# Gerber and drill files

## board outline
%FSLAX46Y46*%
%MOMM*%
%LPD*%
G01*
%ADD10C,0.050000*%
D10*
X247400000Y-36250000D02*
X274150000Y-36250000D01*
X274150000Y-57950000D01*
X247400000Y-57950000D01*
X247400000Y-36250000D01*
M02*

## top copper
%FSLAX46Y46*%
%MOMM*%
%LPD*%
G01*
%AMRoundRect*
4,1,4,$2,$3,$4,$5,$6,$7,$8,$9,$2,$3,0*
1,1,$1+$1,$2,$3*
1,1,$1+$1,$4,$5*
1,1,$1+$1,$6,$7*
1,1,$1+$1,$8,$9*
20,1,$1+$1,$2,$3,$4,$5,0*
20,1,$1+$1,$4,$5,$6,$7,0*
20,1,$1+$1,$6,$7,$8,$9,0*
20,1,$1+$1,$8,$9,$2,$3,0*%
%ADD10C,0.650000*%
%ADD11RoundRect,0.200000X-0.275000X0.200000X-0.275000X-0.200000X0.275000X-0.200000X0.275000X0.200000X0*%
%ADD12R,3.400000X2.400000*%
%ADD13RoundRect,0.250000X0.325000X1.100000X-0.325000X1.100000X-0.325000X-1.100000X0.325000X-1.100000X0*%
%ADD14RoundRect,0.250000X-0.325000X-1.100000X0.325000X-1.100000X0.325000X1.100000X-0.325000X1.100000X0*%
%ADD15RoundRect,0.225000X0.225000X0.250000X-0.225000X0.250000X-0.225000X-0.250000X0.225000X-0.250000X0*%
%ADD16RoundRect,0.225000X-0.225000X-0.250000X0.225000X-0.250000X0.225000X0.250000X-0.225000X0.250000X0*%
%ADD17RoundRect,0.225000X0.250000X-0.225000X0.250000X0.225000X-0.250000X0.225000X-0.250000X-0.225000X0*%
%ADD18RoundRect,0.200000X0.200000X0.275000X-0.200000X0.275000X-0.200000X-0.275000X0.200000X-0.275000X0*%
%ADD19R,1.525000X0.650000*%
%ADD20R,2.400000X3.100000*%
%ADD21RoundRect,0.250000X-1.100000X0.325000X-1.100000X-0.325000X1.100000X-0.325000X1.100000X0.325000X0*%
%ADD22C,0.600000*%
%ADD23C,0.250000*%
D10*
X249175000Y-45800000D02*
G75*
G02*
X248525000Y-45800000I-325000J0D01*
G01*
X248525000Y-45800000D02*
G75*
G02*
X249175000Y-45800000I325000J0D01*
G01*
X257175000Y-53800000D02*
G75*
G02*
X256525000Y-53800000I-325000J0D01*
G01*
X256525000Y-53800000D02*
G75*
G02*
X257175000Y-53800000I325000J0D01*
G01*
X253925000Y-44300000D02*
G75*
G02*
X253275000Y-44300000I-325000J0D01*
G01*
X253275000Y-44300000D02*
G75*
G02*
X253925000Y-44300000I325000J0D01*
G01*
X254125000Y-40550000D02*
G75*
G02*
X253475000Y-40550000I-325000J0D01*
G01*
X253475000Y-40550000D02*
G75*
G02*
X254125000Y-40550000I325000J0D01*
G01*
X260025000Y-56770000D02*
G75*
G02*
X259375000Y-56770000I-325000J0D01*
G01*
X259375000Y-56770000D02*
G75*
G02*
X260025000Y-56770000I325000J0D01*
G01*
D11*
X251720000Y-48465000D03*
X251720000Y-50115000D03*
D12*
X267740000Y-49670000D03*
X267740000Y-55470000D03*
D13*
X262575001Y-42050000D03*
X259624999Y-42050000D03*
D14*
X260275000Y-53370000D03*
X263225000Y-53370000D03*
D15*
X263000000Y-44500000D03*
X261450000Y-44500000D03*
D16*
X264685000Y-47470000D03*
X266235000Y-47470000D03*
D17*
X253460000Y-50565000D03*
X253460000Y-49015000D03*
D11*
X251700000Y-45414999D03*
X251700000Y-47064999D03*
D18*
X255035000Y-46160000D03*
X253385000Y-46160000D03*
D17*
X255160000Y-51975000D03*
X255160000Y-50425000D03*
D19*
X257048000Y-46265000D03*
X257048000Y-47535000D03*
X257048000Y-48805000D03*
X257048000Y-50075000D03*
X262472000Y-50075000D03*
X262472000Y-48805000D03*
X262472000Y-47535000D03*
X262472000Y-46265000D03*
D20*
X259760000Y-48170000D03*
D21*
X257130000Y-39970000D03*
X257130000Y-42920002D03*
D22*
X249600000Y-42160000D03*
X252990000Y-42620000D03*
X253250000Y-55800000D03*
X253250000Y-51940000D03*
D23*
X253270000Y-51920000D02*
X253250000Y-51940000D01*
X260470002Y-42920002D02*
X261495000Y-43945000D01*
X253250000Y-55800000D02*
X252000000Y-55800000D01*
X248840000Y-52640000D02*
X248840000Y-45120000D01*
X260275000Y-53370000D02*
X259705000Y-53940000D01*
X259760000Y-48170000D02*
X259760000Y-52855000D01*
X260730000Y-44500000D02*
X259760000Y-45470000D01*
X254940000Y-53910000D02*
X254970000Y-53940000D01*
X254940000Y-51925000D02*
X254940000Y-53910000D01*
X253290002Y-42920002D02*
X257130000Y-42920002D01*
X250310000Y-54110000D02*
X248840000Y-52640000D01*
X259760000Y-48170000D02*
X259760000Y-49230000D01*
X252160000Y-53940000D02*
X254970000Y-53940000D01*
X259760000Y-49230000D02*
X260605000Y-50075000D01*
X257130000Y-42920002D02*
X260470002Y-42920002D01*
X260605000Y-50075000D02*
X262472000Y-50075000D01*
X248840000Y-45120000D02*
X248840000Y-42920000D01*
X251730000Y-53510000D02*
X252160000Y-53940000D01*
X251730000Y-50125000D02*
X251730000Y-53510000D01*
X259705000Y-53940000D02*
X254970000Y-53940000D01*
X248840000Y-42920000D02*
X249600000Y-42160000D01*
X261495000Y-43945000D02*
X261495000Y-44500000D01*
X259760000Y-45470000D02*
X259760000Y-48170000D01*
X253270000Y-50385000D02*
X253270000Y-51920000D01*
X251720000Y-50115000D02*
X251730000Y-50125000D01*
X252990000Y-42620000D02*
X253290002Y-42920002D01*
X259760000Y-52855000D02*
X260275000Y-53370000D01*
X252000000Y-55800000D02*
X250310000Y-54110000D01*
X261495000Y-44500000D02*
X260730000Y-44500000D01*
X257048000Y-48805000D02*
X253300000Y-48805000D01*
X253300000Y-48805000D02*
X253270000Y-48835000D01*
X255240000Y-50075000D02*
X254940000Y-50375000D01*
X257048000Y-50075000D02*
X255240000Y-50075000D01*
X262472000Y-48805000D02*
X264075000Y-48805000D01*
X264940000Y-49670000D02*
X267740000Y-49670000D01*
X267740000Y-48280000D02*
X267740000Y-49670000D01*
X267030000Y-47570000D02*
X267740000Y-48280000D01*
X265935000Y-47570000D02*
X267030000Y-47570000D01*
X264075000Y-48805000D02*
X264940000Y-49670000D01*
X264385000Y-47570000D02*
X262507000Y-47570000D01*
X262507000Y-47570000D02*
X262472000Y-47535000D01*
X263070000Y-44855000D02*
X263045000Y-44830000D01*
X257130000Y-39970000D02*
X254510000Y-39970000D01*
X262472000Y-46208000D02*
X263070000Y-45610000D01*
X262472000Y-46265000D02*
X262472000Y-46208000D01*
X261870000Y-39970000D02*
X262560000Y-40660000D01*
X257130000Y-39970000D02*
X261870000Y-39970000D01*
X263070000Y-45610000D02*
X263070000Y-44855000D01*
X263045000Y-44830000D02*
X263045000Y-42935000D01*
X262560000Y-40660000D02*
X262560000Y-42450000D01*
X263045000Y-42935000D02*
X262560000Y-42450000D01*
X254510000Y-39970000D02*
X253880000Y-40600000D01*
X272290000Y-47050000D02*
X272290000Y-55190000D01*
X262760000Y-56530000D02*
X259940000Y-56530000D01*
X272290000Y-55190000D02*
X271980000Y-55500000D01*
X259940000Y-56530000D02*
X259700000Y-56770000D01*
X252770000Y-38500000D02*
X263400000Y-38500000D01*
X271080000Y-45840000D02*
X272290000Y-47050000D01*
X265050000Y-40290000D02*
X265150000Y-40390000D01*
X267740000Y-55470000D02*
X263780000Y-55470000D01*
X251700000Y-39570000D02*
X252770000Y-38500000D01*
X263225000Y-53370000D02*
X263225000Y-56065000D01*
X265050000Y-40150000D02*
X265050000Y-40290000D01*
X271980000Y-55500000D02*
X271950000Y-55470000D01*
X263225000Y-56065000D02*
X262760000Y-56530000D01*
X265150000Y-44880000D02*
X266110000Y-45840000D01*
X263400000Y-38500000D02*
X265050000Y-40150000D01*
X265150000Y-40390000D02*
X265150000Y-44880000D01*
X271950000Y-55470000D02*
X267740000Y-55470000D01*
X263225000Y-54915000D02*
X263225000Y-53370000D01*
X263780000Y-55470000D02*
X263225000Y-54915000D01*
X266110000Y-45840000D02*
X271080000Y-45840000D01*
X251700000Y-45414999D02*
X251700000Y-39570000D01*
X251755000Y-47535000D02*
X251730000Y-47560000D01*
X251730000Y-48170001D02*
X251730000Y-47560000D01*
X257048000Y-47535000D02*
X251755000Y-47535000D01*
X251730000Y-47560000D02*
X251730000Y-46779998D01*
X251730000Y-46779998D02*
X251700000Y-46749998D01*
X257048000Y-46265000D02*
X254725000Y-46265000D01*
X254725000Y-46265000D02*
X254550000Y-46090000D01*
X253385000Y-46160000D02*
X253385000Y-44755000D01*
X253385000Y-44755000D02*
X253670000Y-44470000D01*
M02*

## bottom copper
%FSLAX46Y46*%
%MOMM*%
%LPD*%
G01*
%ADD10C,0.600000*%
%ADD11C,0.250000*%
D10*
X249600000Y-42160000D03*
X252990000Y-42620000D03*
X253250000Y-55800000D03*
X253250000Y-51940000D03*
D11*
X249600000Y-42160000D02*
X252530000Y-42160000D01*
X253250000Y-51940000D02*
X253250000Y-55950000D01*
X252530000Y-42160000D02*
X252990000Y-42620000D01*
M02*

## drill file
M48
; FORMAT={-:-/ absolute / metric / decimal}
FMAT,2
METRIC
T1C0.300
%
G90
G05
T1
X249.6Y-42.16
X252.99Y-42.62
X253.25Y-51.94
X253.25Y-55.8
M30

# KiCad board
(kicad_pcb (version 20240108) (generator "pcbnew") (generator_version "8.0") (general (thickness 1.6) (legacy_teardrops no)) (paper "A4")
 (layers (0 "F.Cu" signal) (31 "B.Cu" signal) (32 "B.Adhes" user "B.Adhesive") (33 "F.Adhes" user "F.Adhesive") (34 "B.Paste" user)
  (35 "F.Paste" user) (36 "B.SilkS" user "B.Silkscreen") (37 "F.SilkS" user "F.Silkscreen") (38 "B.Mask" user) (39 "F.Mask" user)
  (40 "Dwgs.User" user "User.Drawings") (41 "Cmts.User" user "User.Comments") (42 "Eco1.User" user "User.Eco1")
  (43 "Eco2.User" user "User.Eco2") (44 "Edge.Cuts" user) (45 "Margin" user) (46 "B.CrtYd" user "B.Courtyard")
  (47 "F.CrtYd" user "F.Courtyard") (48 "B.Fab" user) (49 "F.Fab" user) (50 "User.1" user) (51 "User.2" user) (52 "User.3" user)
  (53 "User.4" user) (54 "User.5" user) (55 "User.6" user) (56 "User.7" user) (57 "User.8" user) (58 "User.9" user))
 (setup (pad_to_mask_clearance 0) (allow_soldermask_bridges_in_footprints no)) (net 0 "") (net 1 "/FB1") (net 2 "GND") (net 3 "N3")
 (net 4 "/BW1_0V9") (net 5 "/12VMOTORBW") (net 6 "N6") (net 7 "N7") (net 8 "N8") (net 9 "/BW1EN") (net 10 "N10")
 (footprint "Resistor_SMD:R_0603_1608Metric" (layer "F.Cu") (at 251.72 49.29 -90)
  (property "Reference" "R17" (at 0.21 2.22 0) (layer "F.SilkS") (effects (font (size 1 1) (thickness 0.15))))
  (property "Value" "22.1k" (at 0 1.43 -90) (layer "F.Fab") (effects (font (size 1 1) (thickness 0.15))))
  (pad "1" smd roundrect (at -0.825 0 270) (size 0.8 0.95) (layers "F.Cu" "F.Paste" "F.Mask") (roundrect_rratio 0.25) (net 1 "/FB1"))
  (pad "2" smd roundrect (at 0.825 0 270) (size 0.8 0.95) (layers "F.Cu" "F.Paste" "F.Mask") (roundrect_rratio 0.25) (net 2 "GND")))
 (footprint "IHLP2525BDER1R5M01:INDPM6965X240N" (layer "F.Cu") (at 267.74 52.57 -90)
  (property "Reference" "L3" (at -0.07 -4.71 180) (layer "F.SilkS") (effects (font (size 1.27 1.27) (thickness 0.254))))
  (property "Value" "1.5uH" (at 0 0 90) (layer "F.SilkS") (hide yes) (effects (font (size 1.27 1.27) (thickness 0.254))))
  (pad "1" smd rect (at -2.9 0 270) (size 2.4 3.4) (layers "F.Cu" "F.Paste" "F.Mask") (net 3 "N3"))
  (pad "2" smd rect (at 2.9 0 270) (size 2.4 3.4) (layers "F.Cu" "F.Paste" "F.Mask") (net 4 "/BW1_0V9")))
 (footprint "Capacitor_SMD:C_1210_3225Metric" (layer "F.Cu") (at 261.1 42.05 180)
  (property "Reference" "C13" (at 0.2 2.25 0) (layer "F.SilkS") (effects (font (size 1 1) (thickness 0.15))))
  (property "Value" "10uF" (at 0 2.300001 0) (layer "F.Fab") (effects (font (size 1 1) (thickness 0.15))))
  (pad "1" smd roundrect (at -1.475001 0 180) (size 1.15 2.7) (layers "F.Cu" "F.Paste" "F.Mask") (roundrect_rratio 0.217391)
   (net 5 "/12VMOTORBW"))
  (pad "2" smd roundrect (at 1.475001 0 180) (size 1.15 2.7) (layers "F.Cu" "F.Paste" "F.Mask") (roundrect_rratio 0.217391) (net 2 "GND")))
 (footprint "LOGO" (layer "F.Cu") (at 268.9 41.65)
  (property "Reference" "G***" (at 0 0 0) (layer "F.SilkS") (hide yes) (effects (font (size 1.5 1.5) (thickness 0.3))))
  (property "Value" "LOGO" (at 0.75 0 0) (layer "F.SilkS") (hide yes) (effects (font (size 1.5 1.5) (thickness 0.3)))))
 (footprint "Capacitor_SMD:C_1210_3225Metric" (layer "F.Cu") (at 261.75 53.37)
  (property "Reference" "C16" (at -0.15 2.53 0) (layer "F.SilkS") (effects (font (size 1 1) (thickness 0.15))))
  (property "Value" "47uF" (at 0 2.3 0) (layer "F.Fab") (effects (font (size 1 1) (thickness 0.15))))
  (pad "1" smd roundrect (at -1.475 0) (size 1.15 2.7) (layers "F.Cu" "F.Paste" "F.Mask") (roundrect_rratio 0.217391) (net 2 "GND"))
  (pad "2" smd roundrect (at 1.475 0) (size 1.15 2.7) (layers "F.Cu" "F.Paste" "F.Mask") (roundrect_rratio 0.217391) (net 4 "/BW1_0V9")))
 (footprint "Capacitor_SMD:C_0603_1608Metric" (layer "F.Cu") (at 262.225 44.5 180)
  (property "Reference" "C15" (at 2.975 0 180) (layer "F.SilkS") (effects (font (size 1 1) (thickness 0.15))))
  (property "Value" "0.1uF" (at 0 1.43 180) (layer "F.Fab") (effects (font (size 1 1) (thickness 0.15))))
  (pad "1" smd roundrect (at -0.775 0 180) (size 0.9 0.95) (layers "F.Cu" "F.Paste" "F.Mask") (roundrect_rratio 0.25) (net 5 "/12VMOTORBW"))
  (pad "2" smd roundrect (at 0.775 0 180) (size 0.9 0.95) (layers "F.Cu" "F.Paste" "F.Mask") (roundrect_rratio 0.25) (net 2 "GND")))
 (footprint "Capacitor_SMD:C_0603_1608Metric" (layer "F.Cu") (at 265.46 47.47)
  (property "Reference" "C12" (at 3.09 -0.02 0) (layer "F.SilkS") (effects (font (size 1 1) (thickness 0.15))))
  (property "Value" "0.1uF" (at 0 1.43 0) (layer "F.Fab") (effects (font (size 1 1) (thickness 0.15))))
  (pad "1" smd roundrect (at -0.775 0) (size 0.9 0.95) (layers "F.Cu" "F.Paste" "F.Mask") (roundrect_rratio 0.25) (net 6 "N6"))
  (pad "2" smd roundrect (at 0.775 0) (size 0.9 0.95) (layers "F.Cu" "F.Paste" "F.Mask") (roundrect_rratio 0.25) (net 3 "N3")))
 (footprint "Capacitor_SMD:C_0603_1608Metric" (layer "F.Cu") (at 253.46 49.79 90)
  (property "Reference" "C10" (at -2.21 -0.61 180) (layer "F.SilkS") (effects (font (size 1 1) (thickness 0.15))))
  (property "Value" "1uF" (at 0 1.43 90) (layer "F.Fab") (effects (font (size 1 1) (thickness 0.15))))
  (pad "1" smd roundrect (at -0.775 0 90) (size 0.9 0.95) (layers "F.Cu" "F.Paste" "F.Mask") (roundrect_rratio 0.25) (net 2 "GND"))
  (pad "2" smd roundrect (at 0.775 0 90) (size 0.9 0.95) (layers "F.Cu" "F.Paste" "F.Mask") (roundrect_rratio 0.25) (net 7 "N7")))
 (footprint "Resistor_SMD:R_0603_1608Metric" (layer "F.Cu") (at 251.7 46.239999 -90)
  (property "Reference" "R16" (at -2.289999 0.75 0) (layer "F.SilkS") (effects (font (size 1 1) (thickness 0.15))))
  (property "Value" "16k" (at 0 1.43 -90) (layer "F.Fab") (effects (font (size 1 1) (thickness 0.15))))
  (pad "1" smd roundrect (at -0.825 0 270) (size 0.8 0.95) (layers "F.Cu" "F.Paste" "F.Mask") (roundrect_rratio 0.25) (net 4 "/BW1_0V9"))
  (pad "2" smd roundrect (at 0.825 0 270) (size 0.8 0.95) (layers "F.Cu" "F.Paste" "F.Mask") (roundrect_rratio 0.25) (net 1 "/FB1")))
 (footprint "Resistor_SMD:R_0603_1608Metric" (layer "F.Cu") (at 254.21 46.16 180)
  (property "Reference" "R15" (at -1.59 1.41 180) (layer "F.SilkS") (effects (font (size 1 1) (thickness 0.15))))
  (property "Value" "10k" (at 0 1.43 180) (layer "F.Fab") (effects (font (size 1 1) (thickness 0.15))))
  (pad "1" smd roundrect (at -0.825 0 180) (size 0.8 0.95) (layers "F.Cu" "F.Paste" "F.Mask") (roundrect_rratio 0.25) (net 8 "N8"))
  (pad "2" smd roundrect (at 0.825 0 180) (size 0.8 0.95) (layers "F.Cu" "F.Paste" "F.Mask") (roundrect_rratio 0.25) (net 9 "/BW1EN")))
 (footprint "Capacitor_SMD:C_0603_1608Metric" (layer "F.Cu") (at 255.16 51.2 90)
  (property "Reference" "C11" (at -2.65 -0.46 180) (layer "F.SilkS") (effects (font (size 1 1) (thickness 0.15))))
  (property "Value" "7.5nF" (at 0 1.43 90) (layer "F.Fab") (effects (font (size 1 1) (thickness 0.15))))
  (pad "1" smd roundrect (at -0.775 0 90) (size 0.9 0.95) (layers "F.Cu" "F.Paste" "F.Mask") (roundrect_rratio 0.25) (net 2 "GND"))
  (pad "2" smd roundrect (at 0.775 0 90) (size 0.9 0.95) (layers "F.Cu" "F.Paste" "F.Mask") (roundrect_rratio 0.25) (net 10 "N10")))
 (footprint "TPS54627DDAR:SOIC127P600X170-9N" (layer "F.Cu") (at 259.76 48.17)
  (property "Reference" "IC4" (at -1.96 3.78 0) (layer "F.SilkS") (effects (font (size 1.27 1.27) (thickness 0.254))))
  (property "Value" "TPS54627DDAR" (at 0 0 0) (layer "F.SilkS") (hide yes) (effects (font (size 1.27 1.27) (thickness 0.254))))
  (pad "1" smd rect (at -2.712 -1.905 90) (size 0.65 1.525) (layers "F.Cu" "F.Paste" "F.Mask") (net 8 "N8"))
  (pad "2" smd rect (at -2.712 -0.635 90) (size 0.65 1.525) (layers "F.Cu" "F.Paste" "F.Mask") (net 1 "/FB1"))
  (pad "3" smd rect (at -2.712 0.635 90) (size 0.65 1.525) (layers "F.Cu" "F.Paste" "F.Mask") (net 7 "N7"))
  (pad "4" smd rect (at -2.712 1.905 90) (size 0.65 1.525) (layers "F.Cu" "F.Paste" "F.Mask") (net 10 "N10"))
  (pad "5" smd rect (at 2.712 1.905 90) (size 0.65 1.525) (layers "F.Cu" "F.Paste" "F.Mask") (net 2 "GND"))
  (pad "6" smd rect (at 2.712 0.635 90) (size 0.65 1.525) (layers "F.Cu" "F.Paste" "F.Mask") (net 3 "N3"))
  (pad "7" smd rect (at 2.712 -0.635 90) (size 0.65 1.525) (layers "F.Cu" "F.Paste" "F.Mask") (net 6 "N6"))
  (pad "8" smd rect (at 2.712 -1.905 90) (size 0.65 1.525) (layers "F.Cu" "F.Paste" "F.Mask") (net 5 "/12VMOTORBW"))
  (pad "9" smd rect (at 0 0) (size 2.4 3.1) (layers "F.Cu" "F.Paste" "F.Mask") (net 2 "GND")))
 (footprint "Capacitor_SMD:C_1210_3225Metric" (layer "F.Cu") (at 257.13 41.445001 -90)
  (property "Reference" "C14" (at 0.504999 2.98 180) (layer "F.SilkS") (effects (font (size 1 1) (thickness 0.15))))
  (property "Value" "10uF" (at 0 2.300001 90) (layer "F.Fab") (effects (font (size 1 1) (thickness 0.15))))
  (pad "1" smd roundrect (at -1.475001 0 270) (size 1.15 2.7) (layers "F.Cu" "F.Paste" "F.Mask") (roundrect_rratio 0.217391)
   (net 5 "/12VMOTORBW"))
  (pad "2" smd roundrect (at 1.475001 0 270) (size 1.15 2.7) (layers "F.Cu" "F.Paste" "F.Mask") (roundrect_rratio 0.217391) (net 2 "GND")))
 (gr_circle (center 248.85 45.8) (end 248.85 45.25) (stroke (width 0.2) (type default)) (fill solid) (layer "F.Cu") (net 2))
 (gr_circle (center 256.85 53.8) (end 256.85 53.25) (stroke (width 0.2) (type default)) (fill solid) (layer "F.Cu") (net 2))
 (gr_circle (center 253.6 44.3) (end 253.6 43.75) (stroke (width 0.2) (type default)) (fill solid) (layer "F.Cu") (net 9))
 (gr_circle (center 253.8 40.55) (end 253.8 40) (stroke (width 0.2) (type default)) (fill solid) (layer "F.Cu") (net 5))
 (gr_circle (center 259.7 56.77) (end 259.7 56.22) (stroke (width 0.2) (type default)) (fill solid) (layer "F.Cu") (net 4))
 (gr_rect (start 247.4 36.25) (end 274.15 57.95) (stroke (width 0.05) (type default)) (fill none) (layer "Edge.Cuts"))
 (segment (start 253.27 51.92) (end 253.25 51.94) (width 0.25) (layer "F.Cu") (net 2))
 (segment (start 260.470002 42.920002) (end 261.495 43.945) (width 0.25) (layer "F.Cu") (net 2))
 (segment (start 253.25 55.8) (end 252 55.8) (width 0.25) (layer "F.Cu") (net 2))
 (segment (start 248.84 52.64) (end 248.84 45.12) (width 0.25) (layer "F.Cu") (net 2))
 (segment (start 260.275 53.37) (end 259.705 53.94) (width 0.25) (layer "F.Cu") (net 2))
 (segment (start 259.76 48.17) (end 259.76 52.855) (width 0.25) (layer "F.Cu") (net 2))
 (segment (start 260.73 44.5) (end 259.76 45.47) (width 0.25) (layer "F.Cu") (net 2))
 (segment (start 254.94 53.91) (end 254.97 53.94) (width 0.25) (layer "F.Cu") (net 2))
 (segment (start 254.94 51.925) (end 254.94 53.91) (width 0.25) (layer "F.Cu") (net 2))
 (segment (start 253.290002 42.920002) (end 257.13 42.920002) (width 0.25) (layer "F.Cu") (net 2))
 (segment (start 250.31 54.11) (end 248.84 52.64) (width 0.25) (layer "F.Cu") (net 2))
 (segment (start 259.76 48.17) (end 259.76 49.23) (width 0.25) (layer "F.Cu") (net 2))
 (segment (start 252.16 53.94) (end 254.97 53.94) (width 0.25) (layer "F.Cu") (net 2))
 (segment (start 259.76 49.23) (end 260.605 50.075) (width 0.25) (layer "F.Cu") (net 2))
 (segment (start 257.13 42.920002) (end 260.470002 42.920002) (width 0.25) (layer "F.Cu") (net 2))
 (segment (start 260.605 50.075) (end 262.472 50.075) (width 0.25) (layer "F.Cu") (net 2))
 (segment (start 248.84 45.12) (end 248.84 42.92) (width 0.25) (layer "F.Cu") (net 2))
 (segment (start 251.73 53.51) (end 252.16 53.94) (width 0.25) (layer "F.Cu") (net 2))
 (segment (start 251.73 50.125) (end 251.73 53.51) (width 0.25) (layer "F.Cu") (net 2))
 (segment (start 259.705 53.94) (end 254.97 53.94) (width 0.25) (layer "F.Cu") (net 2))
 (segment (start 248.84 42.92) (end 249.6 42.16) (width 0.25) (layer "F.Cu") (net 2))
 (segment (start 261.495 43.945) (end 261.495 44.5) (width 0.25) (layer "F.Cu") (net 2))
 (segment (start 259.76 45.47) (end 259.76 48.17) (width 0.25) (layer "F.Cu") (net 2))
 (segment (start 253.27 50.385) (end 253.27 51.92) (width 0.25) (layer "F.Cu") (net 2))
 (segment (start 251.72 50.115) (end 251.73 50.125) (width 0.25) (layer "F.Cu") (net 2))
 (segment (start 252.99 42.62) (end 253.290002 42.920002) (width 0.25) (layer "F.Cu") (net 2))
 (segment (start 259.76 52.855) (end 260.275 53.37) (width 0.25) (layer "F.Cu") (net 2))
 (segment (start 252 55.8) (end 250.31 54.11) (width 0.25) (layer "F.Cu") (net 2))
 (segment (start 261.495 44.5) (end 260.73 44.5) (width 0.25) (layer "F.Cu") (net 2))
 (via (at 249.6 42.16) (size 0.6) (drill 0.3) (layers "F.Cu" "B.Cu") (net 2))
 (via (at 252.99 42.62) (size 0.6) (drill 0.3) (layers "F.Cu" "B.Cu") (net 2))
 (via (at 253.25 55.8) (size 0.6) (drill 0.3) (layers "F.Cu" "B.Cu") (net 2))
 (via (at 253.25 51.94) (size 0.6) (drill 0.3) (layers "F.Cu" "B.Cu") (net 2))
 (segment (start 249.6 42.16) (end 252.53 42.16) (width 0.25) (layer "B.Cu") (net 2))
 (segment (start 253.25 51.94) (end 253.25 55.95) (width 0.25) (layer "B.Cu") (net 2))
 (segment (start 252.53 42.16) (end 252.99 42.62) (width 0.25) (layer "B.Cu") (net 2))
 (segment (start 257.048 48.805) (end 253.3 48.805) (width 0.25) (layer "F.Cu") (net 7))
 (segment (start 253.3 48.805) (end 253.27 48.835) (width 0.25) (layer "F.Cu") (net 7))
 (segment (start 255.24 50.075) (end 254.94 50.375) (width 0.25) (layer "F.Cu") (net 10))
 (segment (start 257.048 50.075) (end 255.24 50.075) (width 0.25) (layer "F.Cu") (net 10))
 (segment (start 262.472 48.805) (end 264.075 48.805) (width 0.25) (layer "F.Cu") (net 3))
 (segment (start 264.94 49.67) (end 267.74 49.67) (width 0.25) (layer "F.Cu") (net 3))
 (segment (start 267.74 48.28) (end 267.74 49.67) (width 0.25) (layer "F.Cu") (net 3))
 (segment (start 267.03 47.57) (end 267.74 48.28) (width 0.25) (layer "F.Cu") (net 3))
 (segment (start 265.935 47.57) (end 267.03 47.57) (width 0.25) (layer "F.Cu") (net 3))
 (segment (start 264.075 48.805) (end 264.94 49.67) (width 0.25) (layer "F.Cu") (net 3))
 (segment (start 264.385 47.57) (end 262.507 47.57) (width 0.25) (layer "F.Cu") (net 6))
 (segment (start 262.507 47.57) (end 262.472 47.535) (width 0.25) (layer "F.Cu") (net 6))
 (segment (start 263.07 44.855) (end 263.045 44.83) (width 0.25) (layer "F.Cu") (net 5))
 (segment (start 257.13 39.97) (end 254.51 39.97) (width 0.25) (layer "F.Cu") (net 5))
 (segment (start 262.472 46.208) (end 263.07 45.61) (width 0.25) (layer "F.Cu") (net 5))
 (segment (start 262.472 46.265) (end 262.472 46.208) (width 0.25) (layer "F.Cu") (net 5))
 (segment (start 261.87 39.97) (end 262.56 40.66) (width 0.25) (layer "F.Cu") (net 5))
 (segment (start 257.13 39.97) (end 261.87 39.97) (width 0.25) (layer "F.Cu") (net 5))
 (segment (start 263.07 45.61) (end 263.07 44.855) (width 0.25) (layer "F.Cu") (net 5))
 (segment (start 263.045 44.83) (end 263.045 42.935) (width 0.25) (layer "F.Cu") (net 5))
 (segment (start 262.56 40.66) (end 262.56 42.45) (width 0.25) (layer "F.Cu") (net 5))
 (segment (start 263.045 42.935) (end 262.56 42.45) (width 0.25) (layer "F.Cu") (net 5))
 (segment (start 254.51 39.97) (end 253.88 40.6) (width 0.25) (layer "F.Cu") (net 5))
 (segment (start 272.29 47.05) (end 272.29 55.19) (width 0.25) (layer "F.Cu") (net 4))
 (segment (start 262.76 56.53) (end 259.94 56.53) (width 0.25) (layer "F.Cu") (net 4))
 (segment (start 272.29 55.19) (end 271.98 55.5) (width 0.25) (layer "F.Cu") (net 4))
 (segment (start 259.94 56.53) (end 259.7 56.77) (width 0.25) (layer "F.Cu") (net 4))
 (segment (start 252.77 38.5) (end 263.4 38.5) (width 0.25) (layer "F.Cu") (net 4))
 (segment (start 271.08 45.84) (end 272.29 47.05) (width 0.25) (layer "F.Cu") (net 4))
 (segment (start 265.05 40.29) (end 265.15 40.39) (width 0.25) (layer "F.Cu") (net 4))
 (segment (start 267.74 55.47) (end 263.78 55.47) (width 0.25) (layer "F.Cu") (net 4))
 (segment (start 251.7 39.57) (end 252.77 38.5) (width 0.25) (layer "F.Cu") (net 4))
 (segment (start 263.225 53.37) (end 263.225 56.065) (width 0.25) (layer "F.Cu") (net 4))
 (segment (start 265.05 40.15) (end 265.05 40.29) (width 0.25) (layer "F.Cu") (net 4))
 (segment (start 271.98 55.5) (end 271.95 55.47) (width 0.25) (layer "F.Cu") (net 4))
 (segment (start 263.225 56.065) (end 262.76 56.53) (width 0.25) (layer "F.Cu") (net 4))
 (segment (start 265.15 44.88) (end 266.11 45.84) (width 0.25) (layer "F.Cu") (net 4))
 (segment (start 263.4 38.5) (end 265.05 40.15) (width 0.25) (layer "F.Cu") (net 4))
 (segment (start 265.15 40.39) (end 265.15 44.88) (width 0.25) (layer "F.Cu") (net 4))
 (segment (start 271.95 55.47) (end 267.74 55.47) (width 0.25) (layer "F.Cu") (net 4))
 (segment (start 263.225 54.915) (end 263.225 53.37) (width 0.25) (layer "F.Cu") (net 4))
 (segment (start 263.78 55.47) (end 263.225 54.915) (width 0.25) (layer "F.Cu") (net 4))
 (segment (start 266.11 45.84) (end 271.08 45.84) (width 0.25) (layer "F.Cu") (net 4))
 (segment (start 251.7 45.414999) (end 251.7 39.57) (width 0.25) (layer "F.Cu") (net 4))
 (segment (start 251.755 47.535) (end 251.73 47.56) (width 0.25) (layer "F.Cu") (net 1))
 (segment (start 251.73 48.170001) (end 251.73 47.56) (width 0.25) (layer "F.Cu") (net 1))
 (segment (start 257.048 47.535) (end 251.755 47.535) (width 0.25) (layer "F.Cu") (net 1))
 (segment (start 251.73 47.56) (end 251.73 46.779998) (width 0.25) (layer "F.Cu") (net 1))
 (segment (start 251.73 46.779998) (end 251.7 46.749998) (width 0.25) (layer "F.Cu") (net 1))
 (segment (start 257.048 46.265) (end 254.725 46.265) (width 0.25) (layer "F.Cu") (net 8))
 (segment (start 254.725 46.265) (end 254.55 46.09) (width 0.25) (layer "F.Cu") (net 8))
 (segment (start 253.385 46.16) (end 253.385 44.755) (width 0.25) (layer "F.Cu") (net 9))
 (segment (start 253.385 44.755) (end 253.67 44.47) (width 0.25) (layer "F.Cu") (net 9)))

